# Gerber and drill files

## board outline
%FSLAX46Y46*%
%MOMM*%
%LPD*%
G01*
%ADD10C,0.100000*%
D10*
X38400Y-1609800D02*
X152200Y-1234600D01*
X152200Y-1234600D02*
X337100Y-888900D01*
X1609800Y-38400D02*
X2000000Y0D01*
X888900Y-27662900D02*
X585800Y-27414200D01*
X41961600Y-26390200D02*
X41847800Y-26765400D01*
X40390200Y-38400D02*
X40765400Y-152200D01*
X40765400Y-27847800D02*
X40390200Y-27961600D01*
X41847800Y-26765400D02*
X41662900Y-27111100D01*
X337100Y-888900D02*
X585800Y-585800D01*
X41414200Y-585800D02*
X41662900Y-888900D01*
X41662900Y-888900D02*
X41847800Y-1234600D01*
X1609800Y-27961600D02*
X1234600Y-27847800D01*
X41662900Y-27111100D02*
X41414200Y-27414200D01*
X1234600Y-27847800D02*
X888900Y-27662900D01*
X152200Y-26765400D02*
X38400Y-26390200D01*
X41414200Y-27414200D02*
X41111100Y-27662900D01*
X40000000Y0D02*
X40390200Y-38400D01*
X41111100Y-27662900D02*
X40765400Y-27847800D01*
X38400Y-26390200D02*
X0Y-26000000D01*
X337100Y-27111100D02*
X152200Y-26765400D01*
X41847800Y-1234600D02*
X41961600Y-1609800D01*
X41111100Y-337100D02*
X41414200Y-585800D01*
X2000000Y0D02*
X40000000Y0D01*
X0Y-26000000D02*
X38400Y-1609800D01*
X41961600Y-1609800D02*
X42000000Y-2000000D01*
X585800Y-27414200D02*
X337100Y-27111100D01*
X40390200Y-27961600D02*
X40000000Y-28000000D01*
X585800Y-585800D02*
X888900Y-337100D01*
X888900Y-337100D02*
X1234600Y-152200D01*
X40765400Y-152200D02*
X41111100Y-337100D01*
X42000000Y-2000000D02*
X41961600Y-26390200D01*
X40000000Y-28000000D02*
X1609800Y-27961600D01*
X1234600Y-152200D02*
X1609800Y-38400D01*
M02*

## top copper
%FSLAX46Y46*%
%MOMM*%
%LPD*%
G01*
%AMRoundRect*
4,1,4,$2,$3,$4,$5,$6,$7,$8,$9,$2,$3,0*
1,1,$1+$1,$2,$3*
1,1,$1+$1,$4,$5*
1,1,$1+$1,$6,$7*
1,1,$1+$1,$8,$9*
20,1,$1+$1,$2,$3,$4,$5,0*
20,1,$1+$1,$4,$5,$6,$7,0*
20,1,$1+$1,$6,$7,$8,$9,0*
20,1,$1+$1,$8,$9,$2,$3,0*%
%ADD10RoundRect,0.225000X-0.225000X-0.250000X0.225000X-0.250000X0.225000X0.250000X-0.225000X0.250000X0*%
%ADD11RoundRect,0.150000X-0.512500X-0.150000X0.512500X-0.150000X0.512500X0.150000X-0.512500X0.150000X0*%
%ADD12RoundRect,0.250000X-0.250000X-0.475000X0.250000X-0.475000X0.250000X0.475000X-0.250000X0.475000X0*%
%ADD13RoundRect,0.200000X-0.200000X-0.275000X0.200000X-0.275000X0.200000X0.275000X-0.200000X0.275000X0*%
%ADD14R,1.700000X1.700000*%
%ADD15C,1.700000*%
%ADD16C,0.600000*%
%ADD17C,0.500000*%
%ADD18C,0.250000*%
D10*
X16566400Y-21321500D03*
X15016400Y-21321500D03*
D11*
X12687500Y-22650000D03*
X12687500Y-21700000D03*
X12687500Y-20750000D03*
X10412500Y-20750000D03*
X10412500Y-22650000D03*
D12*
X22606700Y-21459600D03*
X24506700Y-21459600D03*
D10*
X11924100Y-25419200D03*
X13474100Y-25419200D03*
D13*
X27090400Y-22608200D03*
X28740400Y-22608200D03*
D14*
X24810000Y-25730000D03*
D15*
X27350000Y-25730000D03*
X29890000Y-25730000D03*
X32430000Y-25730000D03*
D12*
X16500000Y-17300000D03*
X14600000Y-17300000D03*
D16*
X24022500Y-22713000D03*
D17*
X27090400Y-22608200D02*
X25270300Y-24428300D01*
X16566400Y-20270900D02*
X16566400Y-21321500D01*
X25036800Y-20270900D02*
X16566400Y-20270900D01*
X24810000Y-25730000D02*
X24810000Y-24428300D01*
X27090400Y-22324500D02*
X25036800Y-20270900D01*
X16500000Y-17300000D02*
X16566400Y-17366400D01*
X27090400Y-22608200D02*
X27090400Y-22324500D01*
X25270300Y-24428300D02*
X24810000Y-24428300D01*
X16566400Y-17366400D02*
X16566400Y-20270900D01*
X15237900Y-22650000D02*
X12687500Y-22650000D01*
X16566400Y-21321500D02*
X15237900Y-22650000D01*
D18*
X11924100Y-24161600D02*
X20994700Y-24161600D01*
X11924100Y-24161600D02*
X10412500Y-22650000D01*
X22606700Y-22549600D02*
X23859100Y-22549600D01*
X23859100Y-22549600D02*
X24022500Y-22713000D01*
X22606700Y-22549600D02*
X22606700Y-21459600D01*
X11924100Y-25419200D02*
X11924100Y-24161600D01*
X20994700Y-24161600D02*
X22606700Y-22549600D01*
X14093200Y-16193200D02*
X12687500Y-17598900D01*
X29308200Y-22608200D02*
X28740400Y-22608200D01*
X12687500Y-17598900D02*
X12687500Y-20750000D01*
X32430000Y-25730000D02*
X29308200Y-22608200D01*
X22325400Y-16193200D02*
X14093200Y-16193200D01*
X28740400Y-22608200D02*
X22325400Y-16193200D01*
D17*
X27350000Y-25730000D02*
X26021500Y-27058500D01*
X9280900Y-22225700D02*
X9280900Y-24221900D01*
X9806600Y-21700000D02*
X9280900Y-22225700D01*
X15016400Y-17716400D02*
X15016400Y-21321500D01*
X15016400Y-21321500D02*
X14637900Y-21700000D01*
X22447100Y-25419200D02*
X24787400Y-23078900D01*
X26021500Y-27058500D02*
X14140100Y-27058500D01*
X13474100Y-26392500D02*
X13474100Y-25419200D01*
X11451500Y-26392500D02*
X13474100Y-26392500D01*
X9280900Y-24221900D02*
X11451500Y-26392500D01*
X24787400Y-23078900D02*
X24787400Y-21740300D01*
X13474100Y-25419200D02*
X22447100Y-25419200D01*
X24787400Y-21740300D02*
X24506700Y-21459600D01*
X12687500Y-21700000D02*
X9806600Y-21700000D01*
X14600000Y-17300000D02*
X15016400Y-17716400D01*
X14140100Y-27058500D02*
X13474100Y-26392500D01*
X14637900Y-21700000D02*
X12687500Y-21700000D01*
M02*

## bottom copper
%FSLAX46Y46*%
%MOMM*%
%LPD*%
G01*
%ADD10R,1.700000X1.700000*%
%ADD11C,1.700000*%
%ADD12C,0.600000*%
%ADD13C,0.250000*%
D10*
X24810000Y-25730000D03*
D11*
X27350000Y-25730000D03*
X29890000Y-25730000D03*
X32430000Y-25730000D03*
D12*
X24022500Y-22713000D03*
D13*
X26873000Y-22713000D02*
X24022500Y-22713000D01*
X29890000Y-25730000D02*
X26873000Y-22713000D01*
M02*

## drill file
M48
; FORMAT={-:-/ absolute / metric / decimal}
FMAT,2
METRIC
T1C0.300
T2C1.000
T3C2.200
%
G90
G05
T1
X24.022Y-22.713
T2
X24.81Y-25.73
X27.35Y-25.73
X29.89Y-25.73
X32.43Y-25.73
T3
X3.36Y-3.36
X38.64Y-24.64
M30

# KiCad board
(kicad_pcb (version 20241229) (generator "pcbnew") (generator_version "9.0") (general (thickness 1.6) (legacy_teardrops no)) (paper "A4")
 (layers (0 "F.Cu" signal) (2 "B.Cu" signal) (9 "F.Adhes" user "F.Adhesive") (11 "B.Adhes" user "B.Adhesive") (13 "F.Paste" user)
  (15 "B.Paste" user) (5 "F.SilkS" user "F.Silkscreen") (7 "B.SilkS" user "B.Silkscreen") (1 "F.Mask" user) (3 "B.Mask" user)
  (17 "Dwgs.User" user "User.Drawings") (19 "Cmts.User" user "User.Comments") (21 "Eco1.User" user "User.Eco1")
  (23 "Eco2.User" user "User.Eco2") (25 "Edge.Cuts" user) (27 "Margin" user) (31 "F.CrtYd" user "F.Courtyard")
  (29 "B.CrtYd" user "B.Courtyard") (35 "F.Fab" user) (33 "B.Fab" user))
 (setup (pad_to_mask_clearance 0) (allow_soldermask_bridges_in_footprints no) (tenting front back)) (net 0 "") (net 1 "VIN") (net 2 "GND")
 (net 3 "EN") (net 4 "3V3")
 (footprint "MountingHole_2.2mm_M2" (layer "F.Cu") (at 3.36 3.36)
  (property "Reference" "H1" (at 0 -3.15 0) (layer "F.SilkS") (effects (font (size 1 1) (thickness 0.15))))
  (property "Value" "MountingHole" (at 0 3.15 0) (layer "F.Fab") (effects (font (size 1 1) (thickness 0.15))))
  (pad "" np_thru_hole circle (at 0 0) (size 2.2 2.2) (drill 2.2) (layers "*.Cu" "*.Mask")))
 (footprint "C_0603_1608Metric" (layer "F.Cu") (at 15.7914 21.3215 180)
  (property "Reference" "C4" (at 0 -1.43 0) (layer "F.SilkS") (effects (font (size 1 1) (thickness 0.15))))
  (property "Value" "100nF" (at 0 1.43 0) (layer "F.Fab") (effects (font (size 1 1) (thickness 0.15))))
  (pad "1" smd roundrect (at -0.775 0) (size 0.9 0.95) (layers "F.Cu" "F.Mask" "F.Paste") (roundrect_rratio 0.25) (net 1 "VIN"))
  (pad "2" smd roundrect (at 0.775 0) (size 0.9 0.95) (layers "F.Cu" "F.Mask" "F.Paste") (roundrect_rratio 0.25) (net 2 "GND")))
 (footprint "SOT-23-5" (layer "F.Cu") (at 11.55 21.7 180)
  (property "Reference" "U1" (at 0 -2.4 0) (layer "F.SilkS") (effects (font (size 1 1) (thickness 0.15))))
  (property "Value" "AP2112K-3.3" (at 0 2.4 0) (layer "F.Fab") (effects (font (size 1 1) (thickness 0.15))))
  (pad "1" smd roundrect (at -1.1375 -0.95) (size 1.325 0.6) (layers "F.Cu" "F.Mask" "F.Paste") (roundrect_rratio 0.25) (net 1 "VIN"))
  (pad "2" smd roundrect (at -1.1375 0) (size 1.325 0.6) (layers "F.Cu" "F.Mask" "F.Paste") (roundrect_rratio 0.25) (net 2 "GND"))
  (pad "3" smd roundrect (at -1.1375 0.95) (size 1.325 0.6) (layers "F.Cu" "F.Mask" "F.Paste") (roundrect_rratio 0.25) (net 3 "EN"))
  (pad "4" smd roundrect (at 1.1375 0.95) (size 1.325 0.6) (layers "F.Cu" "F.Mask" "F.Paste") (roundrect_rratio 0.25))
  (pad "5" smd roundrect (at 1.1375 -0.95) (size 1.325 0.6) (layers "F.Cu" "F.Mask" "F.Paste") (roundrect_rratio 0.25) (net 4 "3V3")))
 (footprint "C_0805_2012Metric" (layer "F.Cu") (at 23.5567 21.4596)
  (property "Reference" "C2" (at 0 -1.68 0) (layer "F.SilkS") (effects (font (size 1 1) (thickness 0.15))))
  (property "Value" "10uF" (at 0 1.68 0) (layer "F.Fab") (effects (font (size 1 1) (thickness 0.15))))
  (pad "1" smd roundrect (at -0.95 0) (size 1 1.45) (layers "F.Cu" "F.Mask" "F.Paste") (roundrect_rratio 0.25) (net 4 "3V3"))
  (pad "2" smd roundrect (at 0.95 0) (size 1 1.45) (layers "F.Cu" "F.Mask" "F.Paste") (roundrect_rratio 0.25) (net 2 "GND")))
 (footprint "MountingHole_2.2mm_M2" (layer "F.Cu") (at 38.64 24.64)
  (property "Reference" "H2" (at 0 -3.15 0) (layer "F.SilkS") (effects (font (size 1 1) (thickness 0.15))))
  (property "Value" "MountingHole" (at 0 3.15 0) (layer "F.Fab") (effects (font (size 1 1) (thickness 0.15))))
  (pad "" np_thru_hole circle (at 0 0) (size 2.2 2.2) (drill 2.2) (layers "*.Cu" "*.Mask")))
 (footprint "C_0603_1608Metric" (layer "F.Cu") (at 12.6991 25.4192)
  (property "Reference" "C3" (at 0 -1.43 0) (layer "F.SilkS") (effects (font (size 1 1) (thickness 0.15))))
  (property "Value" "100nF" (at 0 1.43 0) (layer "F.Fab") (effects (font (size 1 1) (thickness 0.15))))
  (pad "1" smd roundrect (at -0.775 0) (size 0.9 0.95) (layers "F.Cu" "F.Mask" "F.Paste") (roundrect_rratio 0.25) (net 4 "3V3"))
  (pad "2" smd roundrect (at 0.775 0) (size 0.9 0.95) (layers "F.Cu" "F.Mask" "F.Paste") (roundrect_rratio 0.25) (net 2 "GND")))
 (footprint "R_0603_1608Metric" (layer "F.Cu") (at 27.9154 22.6082)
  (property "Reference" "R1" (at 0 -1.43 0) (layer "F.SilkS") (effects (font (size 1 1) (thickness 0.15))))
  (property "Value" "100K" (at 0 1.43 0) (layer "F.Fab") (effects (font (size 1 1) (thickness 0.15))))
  (pad "1" smd roundrect (at -0.825 0) (size 0.8 0.95) (layers "F.Cu" "F.Mask" "F.Paste") (roundrect_rratio 0.25) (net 1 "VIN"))
  (pad "2" smd roundrect (at 0.825 0) (size 0.8 0.95) (layers "F.Cu" "F.Mask" "F.Paste") (roundrect_rratio 0.25) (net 3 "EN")))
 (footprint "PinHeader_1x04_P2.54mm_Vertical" (layer "F.Cu") (at 24.81 25.73 90)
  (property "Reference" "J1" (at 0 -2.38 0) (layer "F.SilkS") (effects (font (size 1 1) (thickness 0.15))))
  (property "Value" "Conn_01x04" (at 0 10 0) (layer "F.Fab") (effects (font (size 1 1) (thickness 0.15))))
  (pad "1" thru_hole rect (at 0 0) (size 1.7 1.7) (drill 1) (layers "*.Cu" "*.Mask") (remove_unused_layers no) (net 1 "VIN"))
  (pad "2" thru_hole circle (at 0 2.54) (size 1.7 1.7) (drill 1) (layers "*.Cu" "*.Mask") (remove_unused_layers no) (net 2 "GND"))
  (pad "3" thru_hole circle (at 0 5.08) (size 1.7 1.7) (drill 1) (layers "*.Cu" "*.Mask") (remove_unused_layers no) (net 4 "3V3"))
  (pad "4" thru_hole circle (at 0 7.62) (size 1.7 1.7) (drill 1) (layers "*.Cu" "*.Mask") (remove_unused_layers no) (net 3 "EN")))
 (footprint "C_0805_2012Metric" (layer "F.Cu") (at 15.55 17.3 180)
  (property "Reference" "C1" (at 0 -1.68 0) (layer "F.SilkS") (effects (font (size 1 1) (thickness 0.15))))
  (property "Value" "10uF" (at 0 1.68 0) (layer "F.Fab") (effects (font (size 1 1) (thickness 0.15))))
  (pad "1" smd roundrect (at -0.95 0) (size 1 1.45) (layers "F.Cu" "F.Mask" "F.Paste") (roundrect_rratio 0.25) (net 1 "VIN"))
  (pad "2" smd roundrect (at 0.95 0) (size 1 1.45) (layers "F.Cu" "F.Mask" "F.Paste") (roundrect_rratio 0.25) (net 2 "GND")))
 (gr_line (start 0.0384 1.6098) (end 0.1522 1.2346) (stroke (width 0.1) (type solid)) (layer "Edge.Cuts"))
 (gr_line (start 0.1522 1.2346) (end 0.3371 0.8889) (stroke (width 0.1) (type solid)) (layer "Edge.Cuts"))
 (gr_line (start 1.6098 0.0384) (end 2 0) (stroke (width 0.1) (type solid)) (layer "Edge.Cuts"))
 (gr_line (start 0.8889 27.6629) (end 0.5858 27.4142) (stroke (width 0.1) (type solid)) (layer "Edge.Cuts"))
 (gr_line (start 41.9616 26.3902) (end 41.8478 26.7654) (stroke (width 0.1) (type solid)) (layer "Edge.Cuts"))
 (gr_line (start 40.3902 0.0384) (end 40.7654 0.1522) (stroke (width 0.1) (type solid)) (layer "Edge.Cuts"))
 (gr_line (start 40.7654 27.8478) (end 40.3902 27.9616) (stroke (width 0.1) (type solid)) (layer "Edge.Cuts"))
 (gr_line (start 41.8478 26.7654) (end 41.6629 27.1111) (stroke (width 0.1) (type solid)) (layer "Edge.Cuts"))
 (gr_line (start 0.3371 0.8889) (end 0.5858 0.5858) (stroke (width 0.1) (type solid)) (layer "Edge.Cuts"))
 (gr_line (start 41.4142 0.5858) (end 41.6629 0.8889) (stroke (width 0.1) (type solid)) (layer "Edge.Cuts"))
 (gr_line (start 41.6629 0.8889) (end 41.8478 1.2346) (stroke (width 0.1) (type solid)) (layer "Edge.Cuts"))
 (gr_line (start 1.6098 27.9616) (end 1.2346 27.8478) (stroke (width 0.1) (type solid)) (layer "Edge.Cuts"))
 (gr_line (start 41.6629 27.1111) (end 41.4142 27.4142) (stroke (width 0.1) (type solid)) (layer "Edge.Cuts"))
 (gr_line (start 1.2346 27.8478) (end 0.8889 27.6629) (stroke (width 0.1) (type solid)) (layer "Edge.Cuts"))
 (gr_line (start 0.1522 26.7654) (end 0.0384 26.3902) (stroke (width 0.1) (type solid)) (layer "Edge.Cuts"))
 (gr_line (start 41.4142 27.4142) (end 41.1111 27.6629) (stroke (width 0.1) (type solid)) (layer "Edge.Cuts"))
 (gr_line (start 40 0) (end 40.3902 0.0384) (stroke (width 0.1) (type solid)) (layer "Edge.Cuts"))
 (gr_line (start 41.1111 27.6629) (end 40.7654 27.8478) (stroke (width 0.1) (type solid)) (layer "Edge.Cuts"))
 (gr_line (start 0.0384 26.3902) (end 0 26) (stroke (width 0.1) (type solid)) (layer "Edge.Cuts"))
 (gr_line (start 0.3371 27.1111) (end 0.1522 26.7654) (stroke (width 0.1) (type solid)) (layer "Edge.Cuts"))
 (gr_line (start 41.8478 1.2346) (end 41.9616 1.6098) (stroke (width 0.1) (type solid)) (layer "Edge.Cuts"))
 (gr_line (start 41.1111 0.3371) (end 41.4142 0.5858) (stroke (width 0.1) (type solid)) (layer "Edge.Cuts"))
 (gr_line (start 2 0) (end 40 0) (stroke (width 0.1) (type solid)) (layer "Edge.Cuts"))
 (gr_line (start 0 26) (end 0.0384 1.6098) (stroke (width 0.1) (type solid)) (layer "Edge.Cuts"))
 (gr_line (start 41.9616 1.6098) (end 42 2) (stroke (width 0.1) (type solid)) (layer "Edge.Cuts"))
 (gr_line (start 0.5858 27.4142) (end 0.3371 27.1111) (stroke (width 0.1) (type solid)) (layer "Edge.Cuts"))
 (gr_line (start 40.3902 27.9616) (end 40 28) (stroke (width 0.1) (type solid)) (layer "Edge.Cuts"))
 (gr_line (start 0.5858 0.5858) (end 0.8889 0.3371) (stroke (width 0.1) (type solid)) (layer "Edge.Cuts"))
 (gr_line (start 0.8889 0.3371) (end 1.2346 0.1522) (stroke (width 0.1) (type solid)) (layer "Edge.Cuts"))
 (gr_line (start 40.7654 0.1522) (end 41.1111 0.3371) (stroke (width 0.1) (type solid)) (layer "Edge.Cuts"))
 (gr_line (start 42 2) (end 41.9616 26.3902) (stroke (width 0.1) (type solid)) (layer "Edge.Cuts"))
 (gr_line (start 40 28) (end 1.6098 27.9616) (stroke (width 0.1) (type solid)) (layer "Edge.Cuts"))
 (gr_line (start 1.2346 0.1522) (end 1.6098 0.0384) (stroke (width 0.1) (type solid)) (layer "Edge.Cuts"))
 (segment (start 27.0904 22.6082) (end 25.2703 24.4283) (width 0.5) (layer "F.Cu") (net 1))
 (segment (start 16.5664 20.2709) (end 16.5664 21.3215) (width 0.5) (layer "F.Cu") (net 1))
 (segment (start 25.0368 20.2709) (end 16.5664 20.2709) (width 0.5) (layer "F.Cu") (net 1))
 (segment (start 24.81 25.73) (end 24.81 24.4283) (width 0.5) (layer "F.Cu") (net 1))
 (segment (start 27.0904 22.3245) (end 25.0368 20.2709) (width 0.5) (layer "F.Cu") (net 1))
 (segment (start 16.5 17.3) (end 16.5664 17.3664) (width 0.5) (layer "F.Cu") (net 1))
 (segment (start 27.0904 22.6082) (end 27.0904 22.3245) (width 0.5) (layer "F.Cu") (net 1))
 (segment (start 25.2703 24.4283) (end 24.81 24.4283) (width 0.5) (layer "F.Cu") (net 1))
 (segment (start 16.5664 17.3664) (end 16.5664 20.2709) (width 0.5) (layer "F.Cu") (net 1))
 (segment (start 15.2379 22.65) (end 12.6875 22.65) (width 0.5) (layer "F.Cu") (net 1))
 (segment (start 16.5664 21.3215) (end 15.2379 22.65) (width 0.5) (layer "F.Cu") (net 1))
 (segment (start 11.9241 24.1616) (end 20.9947 24.1616) (width 0.25) (layer "F.Cu") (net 4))
 (segment (start 11.9241 24.1616) (end 10.4125 22.65) (width 0.25) (layer "F.Cu") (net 4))
 (segment (start 22.6067 22.5496) (end 23.8591 22.5496) (width 0.25) (layer "F.Cu") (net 4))
 (segment (start 23.8591 22.5496) (end 24.0225 22.713) (width 0.25) (layer "F.Cu") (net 4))
 (segment (start 22.6067 22.5496) (end 22.6067 21.4596) (width 0.25) (layer "F.Cu") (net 4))
 (segment (start 11.9241 25.4192) (end 11.9241 24.1616) (width 0.25) (layer "F.Cu") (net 4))
 (segment (start 20.9947 24.1616) (end 22.6067 22.5496) (width 0.25) (layer "F.Cu") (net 4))
 (via (at 24.0225 22.713) (size 0.6) (drill 0.3) (layers "F.Cu" "B.Cu") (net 4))
 (segment (start 26.873 22.713) (end 24.0225 22.713) (width 0.25) (layer "B.Cu") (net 4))
 (segment (start 29.89 25.73) (end 26.873 22.713) (width 0.25) (layer "B.Cu") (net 4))
 (segment (start 14.0932 16.1932) (end 12.6875 17.5989) (width 0.25) (layer "F.Cu") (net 3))
 (segment (start 29.3082 22.6082) (end 28.7404 22.6082) (width 0.25) (layer "F.Cu") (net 3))
 (segment (start 12.6875 17.5989) (end 12.6875 20.75) (width 0.25) (layer "F.Cu") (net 3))
 (segment (start 32.43 25.73) (end 29.3082 22.6082) (width 0.25) (layer "F.Cu") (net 3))
 (segment (start 22.3254 16.1932) (end 14.0932 16.1932) (width 0.25) (layer "F.Cu") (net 3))
 (segment (start 28.7404 22.6082) (end 22.3254 16.1932) (width 0.25) (layer "F.Cu") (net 3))
 (segment (start 27.35 25.73) (end 26.0215 27.0585) (width 0.5) (layer "F.Cu") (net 2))
 (segment (start 9.2809 22.2257) (end 9.2809 24.2219) (width 0.5) (layer "F.Cu") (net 2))
 (segment (start 9.8066 21.7) (end 9.2809 22.2257) (width 0.5) (layer "F.Cu") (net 2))
 (segment (start 15.0164 17.7164) (end 15.0164 21.3215) (width 0.5) (layer "F.Cu") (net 2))
 (segment (start 15.0164 21.3215) (end 14.6379 21.7) (width 0.5) (layer "F.Cu") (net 2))
 (segment (start 22.4471 25.4192) (end 24.7874 23.0789) (width 0.5) (layer "F.Cu") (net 2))
 (segment (start 26.0215 27.0585) (end 14.1401 27.0585) (width 0.5) (layer "F.Cu") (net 2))
 (segment (start 13.4741 26.3925) (end 13.4741 25.4192) (width 0.5) (layer "F.Cu") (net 2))
 (segment (start 11.4515 26.3925) (end 13.4741 26.3925) (width 0.5) (layer "F.Cu") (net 2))
 (segment (start 9.2809 24.2219) (end 11.4515 26.3925) (width 0.5) (layer "F.Cu") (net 2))
 (segment (start 24.7874 23.0789) (end 24.7874 21.7403) (width 0.5) (layer "F.Cu") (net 2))
 (segment (start 13.4741 25.4192) (end 22.4471 25.4192) (width 0.5) (layer "F.Cu") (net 2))
 (segment (start 24.7874 21.7403) (end 24.5067 21.4596) (width 0.5) (layer "F.Cu") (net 2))
 (segment (start 12.6875 21.7) (end 9.8066 21.7) (width 0.5) (layer "F.Cu") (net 2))
 (segment (start 14.6 17.3) (end 15.0164 17.7164) (width 0.5) (layer "F.Cu") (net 2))
 (segment (start 14.1401 27.0585) (end 13.4741 26.3925) (width 0.5) (layer "F.Cu") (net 2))
 (segment (start 14.6379 21.7) (end 12.6875 21.7) (width 0.5) (layer "F.Cu") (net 2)))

